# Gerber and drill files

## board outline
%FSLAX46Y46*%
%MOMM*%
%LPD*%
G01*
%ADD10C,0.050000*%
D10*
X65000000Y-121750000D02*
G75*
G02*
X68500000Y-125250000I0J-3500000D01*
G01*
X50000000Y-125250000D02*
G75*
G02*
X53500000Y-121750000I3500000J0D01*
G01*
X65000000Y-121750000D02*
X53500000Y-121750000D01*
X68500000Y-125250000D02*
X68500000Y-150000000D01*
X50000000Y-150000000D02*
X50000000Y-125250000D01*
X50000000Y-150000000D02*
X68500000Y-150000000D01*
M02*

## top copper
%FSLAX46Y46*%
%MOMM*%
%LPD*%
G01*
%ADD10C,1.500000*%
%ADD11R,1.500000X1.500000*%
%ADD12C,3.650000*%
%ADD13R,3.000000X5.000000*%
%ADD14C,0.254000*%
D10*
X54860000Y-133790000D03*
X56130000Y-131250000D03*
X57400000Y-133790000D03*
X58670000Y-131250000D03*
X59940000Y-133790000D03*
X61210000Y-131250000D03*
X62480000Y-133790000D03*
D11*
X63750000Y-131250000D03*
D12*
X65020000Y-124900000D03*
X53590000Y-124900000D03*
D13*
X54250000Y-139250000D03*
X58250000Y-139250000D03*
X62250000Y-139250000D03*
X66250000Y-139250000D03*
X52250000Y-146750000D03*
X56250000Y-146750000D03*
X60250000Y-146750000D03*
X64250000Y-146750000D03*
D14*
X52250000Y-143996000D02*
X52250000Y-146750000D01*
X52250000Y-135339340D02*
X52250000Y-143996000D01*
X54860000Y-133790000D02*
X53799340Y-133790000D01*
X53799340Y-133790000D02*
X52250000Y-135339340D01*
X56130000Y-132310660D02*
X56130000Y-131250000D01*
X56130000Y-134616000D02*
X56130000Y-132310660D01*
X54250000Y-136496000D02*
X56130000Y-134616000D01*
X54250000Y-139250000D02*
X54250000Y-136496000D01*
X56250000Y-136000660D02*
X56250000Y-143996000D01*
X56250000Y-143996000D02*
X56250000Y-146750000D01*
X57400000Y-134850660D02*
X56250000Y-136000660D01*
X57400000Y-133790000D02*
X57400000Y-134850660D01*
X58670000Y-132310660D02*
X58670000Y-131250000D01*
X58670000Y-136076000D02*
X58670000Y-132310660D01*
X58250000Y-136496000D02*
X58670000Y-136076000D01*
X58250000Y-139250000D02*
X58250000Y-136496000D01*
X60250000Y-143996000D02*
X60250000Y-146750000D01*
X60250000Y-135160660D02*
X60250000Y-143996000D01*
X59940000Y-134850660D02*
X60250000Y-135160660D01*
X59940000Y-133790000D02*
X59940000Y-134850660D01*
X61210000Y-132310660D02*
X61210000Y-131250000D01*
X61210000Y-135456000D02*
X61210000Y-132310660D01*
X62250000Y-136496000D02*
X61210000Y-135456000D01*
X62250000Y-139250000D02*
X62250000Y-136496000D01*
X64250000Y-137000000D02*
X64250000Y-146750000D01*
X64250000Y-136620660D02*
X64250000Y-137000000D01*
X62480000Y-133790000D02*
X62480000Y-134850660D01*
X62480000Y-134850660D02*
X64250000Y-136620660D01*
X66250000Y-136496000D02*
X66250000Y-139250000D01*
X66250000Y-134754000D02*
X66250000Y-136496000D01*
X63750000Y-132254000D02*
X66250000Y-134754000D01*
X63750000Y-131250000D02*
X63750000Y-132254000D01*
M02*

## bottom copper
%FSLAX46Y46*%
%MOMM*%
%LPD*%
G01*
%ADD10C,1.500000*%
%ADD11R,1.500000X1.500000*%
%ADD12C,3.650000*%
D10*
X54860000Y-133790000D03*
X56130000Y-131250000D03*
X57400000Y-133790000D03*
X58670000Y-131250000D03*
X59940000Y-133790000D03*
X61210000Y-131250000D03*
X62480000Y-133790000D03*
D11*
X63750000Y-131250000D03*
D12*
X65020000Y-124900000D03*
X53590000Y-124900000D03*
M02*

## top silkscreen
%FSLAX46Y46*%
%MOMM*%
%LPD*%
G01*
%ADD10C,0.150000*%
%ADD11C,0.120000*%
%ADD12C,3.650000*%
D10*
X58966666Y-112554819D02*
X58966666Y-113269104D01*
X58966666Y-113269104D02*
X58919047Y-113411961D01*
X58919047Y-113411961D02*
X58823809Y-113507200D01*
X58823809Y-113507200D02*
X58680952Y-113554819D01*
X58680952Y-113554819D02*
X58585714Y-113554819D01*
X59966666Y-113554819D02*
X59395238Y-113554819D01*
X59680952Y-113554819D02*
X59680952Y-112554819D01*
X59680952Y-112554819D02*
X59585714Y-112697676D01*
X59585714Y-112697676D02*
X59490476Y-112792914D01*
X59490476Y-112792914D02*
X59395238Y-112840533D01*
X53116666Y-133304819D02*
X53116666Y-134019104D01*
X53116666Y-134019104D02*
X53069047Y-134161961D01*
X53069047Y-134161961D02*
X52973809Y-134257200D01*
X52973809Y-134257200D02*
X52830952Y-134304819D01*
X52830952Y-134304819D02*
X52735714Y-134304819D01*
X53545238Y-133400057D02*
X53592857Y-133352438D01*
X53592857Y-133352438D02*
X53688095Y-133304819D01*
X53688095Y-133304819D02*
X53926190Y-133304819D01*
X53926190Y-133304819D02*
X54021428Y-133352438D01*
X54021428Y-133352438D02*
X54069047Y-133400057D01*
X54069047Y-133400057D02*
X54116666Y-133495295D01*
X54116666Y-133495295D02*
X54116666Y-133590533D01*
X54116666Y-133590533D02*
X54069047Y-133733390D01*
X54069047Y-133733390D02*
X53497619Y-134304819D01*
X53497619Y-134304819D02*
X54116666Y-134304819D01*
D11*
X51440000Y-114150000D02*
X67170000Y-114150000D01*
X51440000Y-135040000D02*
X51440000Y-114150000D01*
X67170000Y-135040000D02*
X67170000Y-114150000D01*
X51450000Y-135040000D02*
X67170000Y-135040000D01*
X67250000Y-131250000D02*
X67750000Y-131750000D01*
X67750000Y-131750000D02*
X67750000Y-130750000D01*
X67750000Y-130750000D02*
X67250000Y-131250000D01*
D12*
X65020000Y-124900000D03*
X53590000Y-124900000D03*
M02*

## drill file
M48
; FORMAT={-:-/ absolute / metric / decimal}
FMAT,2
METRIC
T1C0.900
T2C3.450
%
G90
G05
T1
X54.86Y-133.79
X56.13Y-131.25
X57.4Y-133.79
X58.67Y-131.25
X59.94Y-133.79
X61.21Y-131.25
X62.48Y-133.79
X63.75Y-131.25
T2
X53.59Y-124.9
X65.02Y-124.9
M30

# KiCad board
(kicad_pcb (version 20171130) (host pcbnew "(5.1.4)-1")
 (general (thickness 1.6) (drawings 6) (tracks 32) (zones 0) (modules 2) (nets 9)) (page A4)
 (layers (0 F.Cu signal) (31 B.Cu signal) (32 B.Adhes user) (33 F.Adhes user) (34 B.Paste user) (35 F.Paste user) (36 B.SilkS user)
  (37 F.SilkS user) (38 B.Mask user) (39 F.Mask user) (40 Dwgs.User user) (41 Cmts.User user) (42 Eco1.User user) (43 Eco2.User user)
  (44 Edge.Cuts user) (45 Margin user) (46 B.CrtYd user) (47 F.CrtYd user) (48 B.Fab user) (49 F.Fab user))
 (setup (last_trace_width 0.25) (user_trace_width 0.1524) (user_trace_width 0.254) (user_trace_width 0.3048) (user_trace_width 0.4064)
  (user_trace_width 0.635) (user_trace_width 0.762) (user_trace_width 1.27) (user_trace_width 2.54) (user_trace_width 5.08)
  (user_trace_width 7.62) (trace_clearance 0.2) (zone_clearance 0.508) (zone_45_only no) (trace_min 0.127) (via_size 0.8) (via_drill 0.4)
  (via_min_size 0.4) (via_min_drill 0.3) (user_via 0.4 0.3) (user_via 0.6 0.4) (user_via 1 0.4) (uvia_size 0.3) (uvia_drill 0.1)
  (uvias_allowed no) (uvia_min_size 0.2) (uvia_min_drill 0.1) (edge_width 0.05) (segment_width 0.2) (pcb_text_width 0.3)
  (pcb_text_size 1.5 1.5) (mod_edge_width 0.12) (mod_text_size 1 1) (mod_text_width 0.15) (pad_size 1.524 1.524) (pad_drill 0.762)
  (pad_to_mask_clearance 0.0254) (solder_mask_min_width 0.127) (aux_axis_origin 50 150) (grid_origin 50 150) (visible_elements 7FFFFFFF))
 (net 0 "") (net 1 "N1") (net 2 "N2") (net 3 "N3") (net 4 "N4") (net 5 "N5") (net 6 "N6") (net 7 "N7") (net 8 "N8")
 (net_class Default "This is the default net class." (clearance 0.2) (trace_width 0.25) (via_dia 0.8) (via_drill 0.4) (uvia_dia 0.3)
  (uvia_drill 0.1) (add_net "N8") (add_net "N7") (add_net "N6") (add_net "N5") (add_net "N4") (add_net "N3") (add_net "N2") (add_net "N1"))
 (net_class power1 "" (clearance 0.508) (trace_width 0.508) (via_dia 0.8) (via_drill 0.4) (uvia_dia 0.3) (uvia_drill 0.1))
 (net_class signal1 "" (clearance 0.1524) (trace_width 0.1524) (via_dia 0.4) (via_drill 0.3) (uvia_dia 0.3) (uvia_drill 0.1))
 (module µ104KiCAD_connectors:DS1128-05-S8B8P (layer F.Cu) (at 63.75 131.25 180)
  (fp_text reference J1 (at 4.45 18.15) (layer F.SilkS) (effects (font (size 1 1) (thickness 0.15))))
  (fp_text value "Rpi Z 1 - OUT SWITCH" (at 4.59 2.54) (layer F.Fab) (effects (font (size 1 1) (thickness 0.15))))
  (fp_line (start 12.31 17.1) (end -3.42 17.1) (layer F.SilkS) (width 0.12))
  (fp_line (start 12.31 -3.79) (end 12.31 17.1) (layer F.SilkS) (width 0.12))
  (fp_line (start -3.42 -3.79) (end -3.42 17.1) (layer F.SilkS) (width 0.12))
  (fp_line (start 12.3 -3.79) (end -3.42 -3.79) (layer F.SilkS) (width 0.12))
  (fp_line (start -3.5 0) (end -4 -0.5) (layer F.SilkS) (width 0.12))
  (fp_line (start -4 -0.5) (end -4 0.5) (layer F.SilkS) (width 0.12))
  (fp_line (start -4 0.5) (end -3.5 0) (layer F.SilkS) (width 0.12))
  (pad 8 thru_hole circle (at 8.89 -2.54 180) (size 1.5 1.5) (drill 0.9) (layers *.Cu *.Mask) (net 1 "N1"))
  (pad 7 thru_hole circle (at 7.62 0 180) (size 1.5 1.5) (drill 0.9) (layers *.Cu *.Mask) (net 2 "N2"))
  (pad 6 thru_hole circle (at 6.35 -2.54 180) (size 1.5 1.5) (drill 0.9) (layers *.Cu *.Mask) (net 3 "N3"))
  (pad 5 thru_hole circle (at 5.08 0 180) (size 1.5 1.5) (drill 0.9) (layers *.Cu *.Mask) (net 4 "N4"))
  (pad 4 thru_hole circle (at 3.81 -2.54 180) (size 1.5 1.5) (drill 0.9) (layers *.Cu *.Mask) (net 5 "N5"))
  (pad 3 thru_hole circle (at 2.54 0 180) (size 1.5 1.5) (drill 0.9) (layers *.Cu *.Mask) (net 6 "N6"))
  (pad 2 thru_hole circle (at 1.27 -2.54 180) (size 1.5 1.5) (drill 0.9) (layers *.Cu *.Mask) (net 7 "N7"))
  (pad 1 thru_hole rect (at 0 0 180) (size 1.5 1.5) (drill 0.9) (layers *.Cu *.Mask) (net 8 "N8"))
  (pad "" np_thru_hole circle (at -1.27 6.35 180) (size 3.65 3.65) (drill 3.45) (layers *.Cu *.SilkS *.Mask))
  (pad "" np_thru_hole circle (at 10.16 6.35 180) (size 3.65 3.65) (drill 3.45) (layers *.Cu *.SilkS *.Mask)))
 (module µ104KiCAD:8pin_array (layer F.Cu) (at 54.25 139.25)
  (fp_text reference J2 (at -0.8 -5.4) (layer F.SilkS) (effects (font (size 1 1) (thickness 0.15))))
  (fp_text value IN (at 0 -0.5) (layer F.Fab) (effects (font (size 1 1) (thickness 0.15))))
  (pad 7 smd rect (at 0 0) (size 3 5) (layers F.Cu F.Paste F.Mask) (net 2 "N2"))
  (pad 5 smd rect (at 4 0) (size 3 5) (layers F.Cu F.Paste F.Mask) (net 4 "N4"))
  (pad 3 smd rect (at 8 0) (size 3 5) (layers F.Cu F.Paste F.Mask) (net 6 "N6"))
  (pad 1 smd rect (at 12 0) (size 3 5) (layers F.Cu F.Paste F.Mask) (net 8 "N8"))
  (pad 8 smd rect (at -2 7.5) (size 3 5) (layers F.Cu F.Paste F.Mask) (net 1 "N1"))
  (pad 6 smd rect (at 2 7.5) (size 3 5) (layers F.Cu F.Paste F.Mask) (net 3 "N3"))
  (pad 4 smd rect (at 6 7.5) (size 3 5) (layers F.Cu F.Paste F.Mask) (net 5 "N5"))
  (pad 2 smd rect (at 10 7.5) (size 3 5) (layers F.Cu F.Paste F.Mask) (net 7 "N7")))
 (gr_arc (start 65 125.25) (end 68.5 125.25) (angle -90) (layer Edge.Cuts) (width 0.05))
 (gr_arc (start 53.5 125.25) (end 53.5 121.75) (angle -90) (layer Edge.Cuts) (width 0.05))
 (gr_line (start 65 121.75) (end 53.5 121.75) (layer Edge.Cuts) (width 0.05))
 (gr_line (start 68.5 125.25) (end 68.5 150) (layer Edge.Cuts) (width 0.05))
 (gr_line (start 50 150) (end 50 125.25) (layer Edge.Cuts) (width 0.05))
 (gr_line (start 50 150) (end 68.5 150) (layer Edge.Cuts) (width 0.05))
 (segment (start 52.25 143.996) (end 52.25 146.75) (width 0.254) (layer F.Cu) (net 1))
 (segment (start 52.25 135.33934) (end 52.25 143.996) (width 0.254) (layer F.Cu) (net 1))
 (segment (start 54.86 133.79) (end 53.79934 133.79) (width 0.254) (layer F.Cu) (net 1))
 (segment (start 53.79934 133.79) (end 52.25 135.33934) (width 0.254) (layer F.Cu) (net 1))
 (segment (start 56.13 132.31066) (end 56.13 131.25) (width 0.254) (layer F.Cu) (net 2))
 (segment (start 56.13 134.616) (end 56.13 132.31066) (width 0.254) (layer F.Cu) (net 2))
 (segment (start 54.25 136.496) (end 56.13 134.616) (width 0.254) (layer F.Cu) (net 2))
 (segment (start 54.25 139.25) (end 54.25 136.496) (width 0.254) (layer F.Cu) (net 2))
 (segment (start 56.25 136.00066) (end 56.25 143.996) (width 0.254) (layer F.Cu) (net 3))
 (segment (start 56.25 143.996) (end 56.25 146.75) (width 0.254) (layer F.Cu) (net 3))
 (segment (start 57.4 134.85066) (end 56.25 136.00066) (width 0.254) (layer F.Cu) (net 3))
 (segment (start 57.4 133.79) (end 57.4 134.85066) (width 0.254) (layer F.Cu) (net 3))
 (segment (start 58.67 132.31066) (end 58.67 131.25) (width 0.254) (layer F.Cu) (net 4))
 (segment (start 58.67 136.076) (end 58.67 132.31066) (width 0.254) (layer F.Cu) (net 4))
 (segment (start 58.25 136.496) (end 58.67 136.076) (width 0.254) (layer F.Cu) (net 4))
 (segment (start 58.25 139.25) (end 58.25 136.496) (width 0.254) (layer F.Cu) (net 4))
 (segment (start 60.25 143.996) (end 60.25 146.75) (width 0.254) (layer F.Cu) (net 5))
 (segment (start 60.25 135.16066) (end 60.25 143.996) (width 0.254) (layer F.Cu) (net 5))
 (segment (start 59.94 134.85066) (end 60.25 135.16066) (width 0.254) (layer F.Cu) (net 5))
 (segment (start 59.94 133.79) (end 59.94 134.85066) (width 0.254) (layer F.Cu) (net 5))
 (segment (start 61.21 132.31066) (end 61.21 131.25) (width 0.254) (layer F.Cu) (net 6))
 (segment (start 61.21 135.456) (end 61.21 132.31066) (width 0.254) (layer F.Cu) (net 6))
 (segment (start 62.25 136.496) (end 61.21 135.456) (width 0.254) (layer F.Cu) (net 6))
 (segment (start 62.25 139.25) (end 62.25 136.496) (width 0.254) (layer F.Cu) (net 6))
 (segment (start 64.25 137) (end 64.25 146.75) (width 0.254) (layer F.Cu) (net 7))
 (segment (start 64.25 136.62066) (end 64.25 137) (width 0.254) (layer F.Cu) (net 7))
 (segment (start 62.48 133.79) (end 62.48 134.85066) (width 0.254) (layer F.Cu) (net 7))
 (segment (start 62.48 134.85066) (end 64.25 136.62066) (width 0.254) (layer F.Cu) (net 7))
 (segment (start 66.25 136.496) (end 66.25 139.25) (width 0.254) (layer F.Cu) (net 8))
 (segment (start 66.25 134.754) (end 66.25 136.496) (width 0.254) (layer F.Cu) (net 8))
 (segment (start 63.75 132.254) (end 66.25 134.754) (width 0.254) (layer F.Cu) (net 8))
 (segment (start 63.75 131.25) (end 63.75 132.254) (width 0.254) (layer F.Cu) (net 8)))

